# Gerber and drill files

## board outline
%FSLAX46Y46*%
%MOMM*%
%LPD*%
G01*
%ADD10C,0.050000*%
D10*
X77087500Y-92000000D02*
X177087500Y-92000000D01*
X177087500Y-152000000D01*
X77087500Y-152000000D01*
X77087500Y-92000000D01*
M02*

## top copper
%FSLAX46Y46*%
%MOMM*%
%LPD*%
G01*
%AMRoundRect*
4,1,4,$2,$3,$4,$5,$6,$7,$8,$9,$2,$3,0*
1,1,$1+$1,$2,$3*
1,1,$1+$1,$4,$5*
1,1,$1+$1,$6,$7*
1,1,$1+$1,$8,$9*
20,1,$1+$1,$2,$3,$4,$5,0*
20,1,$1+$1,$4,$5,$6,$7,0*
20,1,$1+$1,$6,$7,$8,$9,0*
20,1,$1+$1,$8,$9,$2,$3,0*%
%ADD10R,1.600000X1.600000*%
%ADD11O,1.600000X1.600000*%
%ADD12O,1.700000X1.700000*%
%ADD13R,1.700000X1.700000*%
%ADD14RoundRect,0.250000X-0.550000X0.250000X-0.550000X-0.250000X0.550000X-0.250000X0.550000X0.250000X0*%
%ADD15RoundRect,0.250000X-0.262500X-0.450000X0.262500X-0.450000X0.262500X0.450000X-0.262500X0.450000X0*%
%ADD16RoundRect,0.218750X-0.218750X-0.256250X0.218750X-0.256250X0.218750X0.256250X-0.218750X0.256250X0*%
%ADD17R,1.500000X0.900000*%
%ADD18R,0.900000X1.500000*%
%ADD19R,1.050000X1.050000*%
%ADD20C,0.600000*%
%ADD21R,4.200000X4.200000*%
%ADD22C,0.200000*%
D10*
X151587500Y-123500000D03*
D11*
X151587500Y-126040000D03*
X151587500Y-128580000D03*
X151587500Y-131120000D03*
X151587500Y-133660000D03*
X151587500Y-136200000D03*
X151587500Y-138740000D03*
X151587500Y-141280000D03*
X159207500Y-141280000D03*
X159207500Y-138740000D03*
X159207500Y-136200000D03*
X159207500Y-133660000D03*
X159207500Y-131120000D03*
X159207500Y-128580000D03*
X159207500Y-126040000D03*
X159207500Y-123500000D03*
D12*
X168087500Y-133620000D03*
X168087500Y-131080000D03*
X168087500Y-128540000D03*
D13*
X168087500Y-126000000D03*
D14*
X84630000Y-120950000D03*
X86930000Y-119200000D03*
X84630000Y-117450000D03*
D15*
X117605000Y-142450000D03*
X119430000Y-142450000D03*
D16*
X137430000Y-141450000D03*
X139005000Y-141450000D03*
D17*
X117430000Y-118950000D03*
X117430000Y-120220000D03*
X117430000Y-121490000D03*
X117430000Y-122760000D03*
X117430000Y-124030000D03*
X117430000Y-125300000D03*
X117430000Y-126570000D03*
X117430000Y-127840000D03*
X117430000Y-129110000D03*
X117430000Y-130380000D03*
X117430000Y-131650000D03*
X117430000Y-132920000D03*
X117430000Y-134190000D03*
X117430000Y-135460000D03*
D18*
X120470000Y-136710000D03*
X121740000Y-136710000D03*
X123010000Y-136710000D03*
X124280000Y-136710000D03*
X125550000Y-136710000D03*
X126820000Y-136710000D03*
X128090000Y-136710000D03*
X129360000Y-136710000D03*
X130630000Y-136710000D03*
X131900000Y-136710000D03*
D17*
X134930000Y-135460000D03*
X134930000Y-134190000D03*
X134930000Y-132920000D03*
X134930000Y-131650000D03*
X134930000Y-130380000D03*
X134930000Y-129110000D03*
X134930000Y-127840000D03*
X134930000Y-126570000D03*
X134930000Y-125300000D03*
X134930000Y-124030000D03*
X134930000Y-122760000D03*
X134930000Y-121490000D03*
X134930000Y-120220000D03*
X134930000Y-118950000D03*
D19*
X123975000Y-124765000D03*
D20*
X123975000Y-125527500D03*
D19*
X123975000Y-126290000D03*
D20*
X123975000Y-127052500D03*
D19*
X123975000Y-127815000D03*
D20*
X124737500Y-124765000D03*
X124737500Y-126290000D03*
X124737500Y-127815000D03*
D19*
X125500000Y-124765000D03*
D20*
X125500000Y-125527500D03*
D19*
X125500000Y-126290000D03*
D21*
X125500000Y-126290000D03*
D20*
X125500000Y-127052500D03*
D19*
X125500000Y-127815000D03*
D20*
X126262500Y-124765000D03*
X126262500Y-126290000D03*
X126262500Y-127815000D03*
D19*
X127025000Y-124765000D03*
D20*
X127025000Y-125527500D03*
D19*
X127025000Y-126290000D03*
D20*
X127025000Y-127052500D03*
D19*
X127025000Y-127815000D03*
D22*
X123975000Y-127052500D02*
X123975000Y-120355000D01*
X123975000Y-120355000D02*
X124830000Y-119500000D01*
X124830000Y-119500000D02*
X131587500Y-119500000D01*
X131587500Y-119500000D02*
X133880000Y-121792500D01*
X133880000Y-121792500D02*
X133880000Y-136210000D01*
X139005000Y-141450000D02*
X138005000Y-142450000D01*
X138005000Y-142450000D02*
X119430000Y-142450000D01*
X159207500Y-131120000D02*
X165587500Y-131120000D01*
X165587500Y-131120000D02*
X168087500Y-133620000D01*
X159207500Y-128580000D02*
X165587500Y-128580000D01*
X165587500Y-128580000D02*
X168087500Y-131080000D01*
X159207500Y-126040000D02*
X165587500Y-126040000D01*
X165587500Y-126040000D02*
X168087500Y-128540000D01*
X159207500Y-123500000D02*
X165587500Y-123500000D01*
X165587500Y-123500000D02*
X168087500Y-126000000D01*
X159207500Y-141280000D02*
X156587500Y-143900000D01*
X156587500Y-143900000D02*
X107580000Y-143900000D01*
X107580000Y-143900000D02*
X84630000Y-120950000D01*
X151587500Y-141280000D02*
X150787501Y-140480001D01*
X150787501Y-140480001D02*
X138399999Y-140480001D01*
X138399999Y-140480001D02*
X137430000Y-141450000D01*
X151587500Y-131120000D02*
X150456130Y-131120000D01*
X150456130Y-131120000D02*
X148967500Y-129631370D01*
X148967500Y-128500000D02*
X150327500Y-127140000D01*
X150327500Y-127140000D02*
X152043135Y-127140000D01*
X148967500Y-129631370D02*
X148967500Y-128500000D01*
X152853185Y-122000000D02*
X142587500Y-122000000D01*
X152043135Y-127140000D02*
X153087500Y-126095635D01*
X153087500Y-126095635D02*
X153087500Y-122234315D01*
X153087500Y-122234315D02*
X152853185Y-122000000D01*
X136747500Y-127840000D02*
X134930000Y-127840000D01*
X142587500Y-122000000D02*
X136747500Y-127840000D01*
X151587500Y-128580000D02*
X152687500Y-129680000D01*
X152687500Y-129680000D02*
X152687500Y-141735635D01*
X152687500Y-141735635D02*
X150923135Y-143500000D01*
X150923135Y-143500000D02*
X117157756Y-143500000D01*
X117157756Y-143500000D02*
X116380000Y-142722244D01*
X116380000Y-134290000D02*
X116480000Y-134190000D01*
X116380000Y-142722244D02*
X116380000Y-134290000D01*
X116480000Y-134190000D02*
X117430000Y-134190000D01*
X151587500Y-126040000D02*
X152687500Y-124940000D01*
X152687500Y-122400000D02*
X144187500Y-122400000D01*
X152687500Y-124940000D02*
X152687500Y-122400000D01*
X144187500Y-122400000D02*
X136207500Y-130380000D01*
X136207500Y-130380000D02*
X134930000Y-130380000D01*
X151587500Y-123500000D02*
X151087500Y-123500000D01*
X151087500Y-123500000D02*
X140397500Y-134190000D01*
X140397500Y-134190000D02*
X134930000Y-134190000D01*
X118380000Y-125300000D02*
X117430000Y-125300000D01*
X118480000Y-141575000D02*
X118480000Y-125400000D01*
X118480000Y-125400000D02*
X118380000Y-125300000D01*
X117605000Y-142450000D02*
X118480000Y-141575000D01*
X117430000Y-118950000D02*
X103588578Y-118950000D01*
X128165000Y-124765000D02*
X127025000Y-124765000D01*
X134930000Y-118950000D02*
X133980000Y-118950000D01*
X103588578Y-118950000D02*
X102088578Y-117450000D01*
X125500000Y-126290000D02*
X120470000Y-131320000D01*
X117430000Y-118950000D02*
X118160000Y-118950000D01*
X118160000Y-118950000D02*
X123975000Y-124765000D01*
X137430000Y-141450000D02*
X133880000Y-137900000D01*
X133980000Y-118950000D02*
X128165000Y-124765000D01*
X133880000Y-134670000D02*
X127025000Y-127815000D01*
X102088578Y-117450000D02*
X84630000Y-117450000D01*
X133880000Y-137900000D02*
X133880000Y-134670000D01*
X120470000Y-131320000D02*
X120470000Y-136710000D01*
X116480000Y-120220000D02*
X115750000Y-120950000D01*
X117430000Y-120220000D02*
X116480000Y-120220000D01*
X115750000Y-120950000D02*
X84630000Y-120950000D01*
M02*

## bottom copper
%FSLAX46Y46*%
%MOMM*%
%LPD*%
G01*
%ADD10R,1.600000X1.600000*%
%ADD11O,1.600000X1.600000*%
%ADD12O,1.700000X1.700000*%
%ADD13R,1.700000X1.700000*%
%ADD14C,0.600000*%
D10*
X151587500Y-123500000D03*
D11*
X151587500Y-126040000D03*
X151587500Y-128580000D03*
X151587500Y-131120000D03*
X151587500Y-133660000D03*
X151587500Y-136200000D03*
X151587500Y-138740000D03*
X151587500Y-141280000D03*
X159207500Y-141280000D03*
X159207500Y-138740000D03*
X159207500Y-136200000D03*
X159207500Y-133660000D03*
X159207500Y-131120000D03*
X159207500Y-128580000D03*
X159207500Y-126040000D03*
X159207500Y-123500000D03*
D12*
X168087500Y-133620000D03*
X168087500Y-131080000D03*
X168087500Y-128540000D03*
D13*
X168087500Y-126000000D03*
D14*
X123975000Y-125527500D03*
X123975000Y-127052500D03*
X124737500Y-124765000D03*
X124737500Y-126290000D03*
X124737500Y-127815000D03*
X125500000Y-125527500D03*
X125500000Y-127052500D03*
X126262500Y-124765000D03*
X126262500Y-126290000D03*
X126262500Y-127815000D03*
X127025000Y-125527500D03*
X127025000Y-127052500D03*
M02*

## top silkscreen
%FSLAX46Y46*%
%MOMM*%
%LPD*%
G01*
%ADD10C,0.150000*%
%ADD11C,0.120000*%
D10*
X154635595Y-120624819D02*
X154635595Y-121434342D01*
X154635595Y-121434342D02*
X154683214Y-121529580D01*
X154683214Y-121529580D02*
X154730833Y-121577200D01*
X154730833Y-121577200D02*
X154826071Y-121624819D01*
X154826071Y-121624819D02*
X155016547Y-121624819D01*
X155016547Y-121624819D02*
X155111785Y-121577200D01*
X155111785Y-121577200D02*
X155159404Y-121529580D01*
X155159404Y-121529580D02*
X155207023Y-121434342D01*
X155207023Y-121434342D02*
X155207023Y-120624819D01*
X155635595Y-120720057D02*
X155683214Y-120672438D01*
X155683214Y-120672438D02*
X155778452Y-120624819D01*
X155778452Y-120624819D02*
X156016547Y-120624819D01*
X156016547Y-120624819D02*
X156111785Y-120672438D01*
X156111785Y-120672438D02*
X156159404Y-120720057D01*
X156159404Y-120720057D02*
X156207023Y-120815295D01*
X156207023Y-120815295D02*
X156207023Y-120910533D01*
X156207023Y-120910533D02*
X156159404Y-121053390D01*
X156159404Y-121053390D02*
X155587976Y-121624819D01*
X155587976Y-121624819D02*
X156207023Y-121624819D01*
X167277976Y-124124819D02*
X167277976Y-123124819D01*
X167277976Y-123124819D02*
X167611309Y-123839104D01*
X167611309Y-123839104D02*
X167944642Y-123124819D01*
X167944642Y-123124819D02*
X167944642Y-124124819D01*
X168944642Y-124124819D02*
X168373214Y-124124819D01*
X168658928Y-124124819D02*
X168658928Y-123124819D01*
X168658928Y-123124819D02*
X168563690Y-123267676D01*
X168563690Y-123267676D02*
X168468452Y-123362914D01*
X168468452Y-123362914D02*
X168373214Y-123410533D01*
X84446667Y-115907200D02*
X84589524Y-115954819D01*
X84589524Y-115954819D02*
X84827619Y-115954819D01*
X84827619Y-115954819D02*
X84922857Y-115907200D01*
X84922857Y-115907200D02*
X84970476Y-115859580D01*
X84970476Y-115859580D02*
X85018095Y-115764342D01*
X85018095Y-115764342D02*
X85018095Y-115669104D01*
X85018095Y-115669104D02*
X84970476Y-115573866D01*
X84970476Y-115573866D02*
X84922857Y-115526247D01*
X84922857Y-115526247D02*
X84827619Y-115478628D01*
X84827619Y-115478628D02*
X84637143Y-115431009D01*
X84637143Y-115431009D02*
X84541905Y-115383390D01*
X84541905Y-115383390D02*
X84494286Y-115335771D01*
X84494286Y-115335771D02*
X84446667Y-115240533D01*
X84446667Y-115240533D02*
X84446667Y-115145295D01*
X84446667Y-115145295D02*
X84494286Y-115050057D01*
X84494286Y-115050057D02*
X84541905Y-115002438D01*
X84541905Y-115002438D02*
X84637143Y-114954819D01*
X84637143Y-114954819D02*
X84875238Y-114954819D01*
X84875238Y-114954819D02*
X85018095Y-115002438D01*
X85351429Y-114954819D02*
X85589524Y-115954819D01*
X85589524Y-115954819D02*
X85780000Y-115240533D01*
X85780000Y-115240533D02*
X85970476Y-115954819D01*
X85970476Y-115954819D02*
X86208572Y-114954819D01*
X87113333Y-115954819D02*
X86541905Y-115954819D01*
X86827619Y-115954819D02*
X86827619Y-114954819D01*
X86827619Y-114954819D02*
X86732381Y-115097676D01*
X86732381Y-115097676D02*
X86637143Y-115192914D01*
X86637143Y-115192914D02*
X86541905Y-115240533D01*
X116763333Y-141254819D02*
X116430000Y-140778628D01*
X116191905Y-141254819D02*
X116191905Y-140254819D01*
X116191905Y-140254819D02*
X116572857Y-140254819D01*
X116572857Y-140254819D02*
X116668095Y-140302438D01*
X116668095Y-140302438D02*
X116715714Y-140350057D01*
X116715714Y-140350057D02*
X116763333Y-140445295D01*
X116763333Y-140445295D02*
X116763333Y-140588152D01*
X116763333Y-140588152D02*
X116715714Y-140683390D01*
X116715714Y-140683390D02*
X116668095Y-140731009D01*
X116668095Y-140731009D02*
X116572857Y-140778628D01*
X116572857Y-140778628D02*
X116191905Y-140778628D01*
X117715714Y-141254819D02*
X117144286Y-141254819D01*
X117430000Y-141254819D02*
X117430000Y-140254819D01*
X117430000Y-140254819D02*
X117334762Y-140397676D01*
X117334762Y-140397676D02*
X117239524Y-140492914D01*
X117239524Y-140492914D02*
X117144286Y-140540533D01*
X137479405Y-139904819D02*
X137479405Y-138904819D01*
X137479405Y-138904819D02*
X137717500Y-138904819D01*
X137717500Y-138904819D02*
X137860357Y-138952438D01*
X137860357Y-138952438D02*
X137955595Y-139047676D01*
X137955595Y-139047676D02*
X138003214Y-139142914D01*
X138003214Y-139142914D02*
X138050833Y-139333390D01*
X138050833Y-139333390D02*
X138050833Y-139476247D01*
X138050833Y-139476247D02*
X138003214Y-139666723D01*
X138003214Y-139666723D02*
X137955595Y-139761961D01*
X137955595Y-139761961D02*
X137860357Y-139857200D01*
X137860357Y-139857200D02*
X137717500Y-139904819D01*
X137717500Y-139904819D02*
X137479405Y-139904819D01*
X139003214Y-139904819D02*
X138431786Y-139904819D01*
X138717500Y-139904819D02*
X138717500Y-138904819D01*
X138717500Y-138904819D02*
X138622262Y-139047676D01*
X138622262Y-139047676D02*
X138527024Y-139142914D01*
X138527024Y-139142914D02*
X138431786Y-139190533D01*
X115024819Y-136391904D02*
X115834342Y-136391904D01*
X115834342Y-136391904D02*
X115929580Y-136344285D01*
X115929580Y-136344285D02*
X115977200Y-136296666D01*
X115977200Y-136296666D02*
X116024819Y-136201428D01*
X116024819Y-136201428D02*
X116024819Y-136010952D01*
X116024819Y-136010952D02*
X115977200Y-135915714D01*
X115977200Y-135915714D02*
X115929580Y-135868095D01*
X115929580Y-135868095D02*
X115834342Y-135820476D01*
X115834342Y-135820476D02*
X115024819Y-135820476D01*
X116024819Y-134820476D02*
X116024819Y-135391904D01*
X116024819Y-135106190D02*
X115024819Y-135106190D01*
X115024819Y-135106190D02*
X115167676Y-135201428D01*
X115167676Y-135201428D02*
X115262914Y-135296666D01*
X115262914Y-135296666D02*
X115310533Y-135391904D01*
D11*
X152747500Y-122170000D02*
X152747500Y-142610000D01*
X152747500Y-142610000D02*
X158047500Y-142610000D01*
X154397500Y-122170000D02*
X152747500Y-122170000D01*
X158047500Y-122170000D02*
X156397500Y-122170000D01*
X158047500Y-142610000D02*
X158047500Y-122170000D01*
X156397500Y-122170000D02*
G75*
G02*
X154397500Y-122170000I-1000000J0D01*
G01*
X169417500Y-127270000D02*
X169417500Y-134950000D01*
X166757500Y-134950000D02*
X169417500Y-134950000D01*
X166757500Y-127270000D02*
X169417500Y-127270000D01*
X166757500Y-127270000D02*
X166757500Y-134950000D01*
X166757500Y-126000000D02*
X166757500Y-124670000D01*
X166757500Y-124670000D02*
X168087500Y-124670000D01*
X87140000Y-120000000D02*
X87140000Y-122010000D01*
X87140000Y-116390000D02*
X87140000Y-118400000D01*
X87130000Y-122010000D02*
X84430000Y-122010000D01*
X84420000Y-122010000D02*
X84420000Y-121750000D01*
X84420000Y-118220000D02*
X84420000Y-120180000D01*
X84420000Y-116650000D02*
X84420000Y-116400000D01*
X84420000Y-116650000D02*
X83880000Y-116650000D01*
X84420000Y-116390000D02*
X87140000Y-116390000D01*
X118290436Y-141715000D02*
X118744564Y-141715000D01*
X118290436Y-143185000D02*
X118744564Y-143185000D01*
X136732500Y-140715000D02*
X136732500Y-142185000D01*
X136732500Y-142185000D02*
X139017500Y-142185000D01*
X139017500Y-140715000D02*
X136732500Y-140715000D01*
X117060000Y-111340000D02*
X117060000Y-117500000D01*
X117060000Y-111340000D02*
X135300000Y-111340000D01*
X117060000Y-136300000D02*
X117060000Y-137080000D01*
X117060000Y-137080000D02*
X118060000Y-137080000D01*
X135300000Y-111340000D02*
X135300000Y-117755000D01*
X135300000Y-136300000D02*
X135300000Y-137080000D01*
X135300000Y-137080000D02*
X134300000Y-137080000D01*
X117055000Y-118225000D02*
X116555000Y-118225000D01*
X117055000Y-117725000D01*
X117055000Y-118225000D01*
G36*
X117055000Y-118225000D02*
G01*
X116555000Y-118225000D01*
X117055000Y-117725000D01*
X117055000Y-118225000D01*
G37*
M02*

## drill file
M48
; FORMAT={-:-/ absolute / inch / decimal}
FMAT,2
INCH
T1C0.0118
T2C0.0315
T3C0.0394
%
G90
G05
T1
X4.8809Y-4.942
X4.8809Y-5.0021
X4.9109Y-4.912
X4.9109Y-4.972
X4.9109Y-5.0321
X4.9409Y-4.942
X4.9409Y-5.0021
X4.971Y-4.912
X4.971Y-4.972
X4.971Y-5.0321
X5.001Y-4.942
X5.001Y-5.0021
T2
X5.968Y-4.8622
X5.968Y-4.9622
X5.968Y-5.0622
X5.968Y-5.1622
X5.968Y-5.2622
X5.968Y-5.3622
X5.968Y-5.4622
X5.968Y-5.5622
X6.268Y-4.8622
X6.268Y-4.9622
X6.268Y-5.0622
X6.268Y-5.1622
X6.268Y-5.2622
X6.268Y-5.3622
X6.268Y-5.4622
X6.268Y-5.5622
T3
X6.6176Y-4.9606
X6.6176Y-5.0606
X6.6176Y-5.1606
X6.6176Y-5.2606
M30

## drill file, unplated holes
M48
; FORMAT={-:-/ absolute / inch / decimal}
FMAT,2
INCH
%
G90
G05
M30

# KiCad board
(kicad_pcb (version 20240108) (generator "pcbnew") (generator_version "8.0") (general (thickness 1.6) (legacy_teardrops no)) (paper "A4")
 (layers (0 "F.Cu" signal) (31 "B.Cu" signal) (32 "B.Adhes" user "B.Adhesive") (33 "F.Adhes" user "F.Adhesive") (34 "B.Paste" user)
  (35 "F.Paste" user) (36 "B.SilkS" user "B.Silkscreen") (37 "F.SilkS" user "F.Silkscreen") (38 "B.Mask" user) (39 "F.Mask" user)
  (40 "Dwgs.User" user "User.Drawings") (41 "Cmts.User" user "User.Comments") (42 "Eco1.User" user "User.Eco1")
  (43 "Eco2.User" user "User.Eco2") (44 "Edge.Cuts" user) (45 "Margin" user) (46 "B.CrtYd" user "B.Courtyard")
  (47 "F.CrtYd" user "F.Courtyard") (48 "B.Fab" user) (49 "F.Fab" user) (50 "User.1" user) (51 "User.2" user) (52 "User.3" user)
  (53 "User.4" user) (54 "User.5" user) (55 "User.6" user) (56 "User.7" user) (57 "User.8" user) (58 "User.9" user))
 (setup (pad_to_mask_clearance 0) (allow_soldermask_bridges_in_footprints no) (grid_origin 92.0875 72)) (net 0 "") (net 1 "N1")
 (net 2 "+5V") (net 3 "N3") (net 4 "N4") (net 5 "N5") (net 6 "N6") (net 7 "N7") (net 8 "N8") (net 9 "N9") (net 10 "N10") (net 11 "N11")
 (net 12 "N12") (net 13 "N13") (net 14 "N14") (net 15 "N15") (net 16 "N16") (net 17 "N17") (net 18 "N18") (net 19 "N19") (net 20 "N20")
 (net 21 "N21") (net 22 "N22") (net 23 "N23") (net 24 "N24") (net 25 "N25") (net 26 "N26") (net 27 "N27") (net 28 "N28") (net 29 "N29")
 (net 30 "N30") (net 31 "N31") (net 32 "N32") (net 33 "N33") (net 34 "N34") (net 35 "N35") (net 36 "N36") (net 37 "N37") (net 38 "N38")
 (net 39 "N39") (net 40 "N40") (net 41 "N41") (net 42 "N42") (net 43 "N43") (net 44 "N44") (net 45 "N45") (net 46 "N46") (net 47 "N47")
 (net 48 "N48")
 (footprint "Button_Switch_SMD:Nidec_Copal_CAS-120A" (layer "F.Cu") (at 85.78 119.2)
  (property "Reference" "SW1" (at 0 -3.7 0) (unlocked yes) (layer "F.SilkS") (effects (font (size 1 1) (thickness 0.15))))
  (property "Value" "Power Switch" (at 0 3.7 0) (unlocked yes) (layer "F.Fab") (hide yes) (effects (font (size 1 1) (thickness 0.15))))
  (fp_line (start -1.36 -2.81) (end 1.36 -2.81) (stroke (width 0.12) (type solid)) (layer "F.SilkS"))
  (fp_line (start -1.36 -2.55) (end -1.9 -2.55) (stroke (width 0.12) (type default)) (layer "F.SilkS"))
  (fp_line (start -1.36 -2.55) (end -1.36 -2.8) (stroke (width 0.12) (type solid)) (layer "F.SilkS"))
  (fp_line (start -1.36 -0.98) (end -1.36 0.98) (stroke (width 0.12) (type solid)) (layer "F.SilkS"))
  (fp_line (start -1.36 2.81) (end -1.36 2.55) (stroke (width 0.12) (type solid)) (layer "F.SilkS"))
  (fp_line (start 1.35 2.81) (end -1.35 2.81) (stroke (width 0.12) (type solid)) (layer "F.SilkS"))
  (fp_line (start 1.36 -2.81) (end 1.36 -0.8) (stroke (width 0.12) (type solid)) (layer "F.SilkS"))
  (fp_line (start 1.36 0.8) (end 1.36 2.81) (stroke (width 0.12) (type solid)) (layer "F.SilkS"))
  (pad "1" smd roundrect (at -1.15 -1.75 270) (size 1 1.6) (layers "F.Cu" "F.Paste" "F.Mask") (roundrect_rratio 0.25) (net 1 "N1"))
  (pad "2" smd roundrect (at 1.15 0 270) (size 1 1.6) (layers "F.Cu" "F.Paste" "F.Mask") (roundrect_rratio 0.25) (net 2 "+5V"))
  (pad "3" smd roundrect (at -1.15 1.75 270) (size 1 1.6) (layers "F.Cu" "F.Paste" "F.Mask") (roundrect_rratio 0.25) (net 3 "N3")))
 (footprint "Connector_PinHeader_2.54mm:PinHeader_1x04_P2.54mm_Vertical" (layer "F.Cu") (at 168.0875 126)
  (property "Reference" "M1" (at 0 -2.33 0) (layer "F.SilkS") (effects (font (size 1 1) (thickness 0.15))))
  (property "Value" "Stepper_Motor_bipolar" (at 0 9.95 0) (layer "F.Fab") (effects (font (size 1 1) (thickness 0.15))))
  (fp_line (start -1.33 -1.33) (end 0 -1.33) (stroke (width 0.12) (type solid)) (layer "F.SilkS"))
  (fp_line (start -1.33 0) (end -1.33 -1.33) (stroke (width 0.12) (type solid)) (layer "F.SilkS"))
  (fp_line (start -1.33 1.27) (end -1.33 8.95) (stroke (width 0.12) (type solid)) (layer "F.SilkS"))
  (fp_line (start -1.33 1.27) (end 1.33 1.27) (stroke (width 0.12) (type solid)) (layer "F.SilkS"))
  (fp_line (start -1.33 8.95) (end 1.33 8.95) (stroke (width 0.12) (type solid)) (layer "F.SilkS"))
  (fp_line (start 1.33 1.27) (end 1.33 8.95) (stroke (width 0.12) (type solid)) (layer "F.SilkS"))
  (pad "1" thru_hole rect (at 0 0) (size 1.7 1.7) (drill 1) (layers "*.Cu" "*.Mask") (remove_unused_layers no) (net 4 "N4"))
  (pad "2" thru_hole oval (at 0 2.54) (size 1.7 1.7) (drill 1) (layers "*.Cu" "*.Mask") (remove_unused_layers no) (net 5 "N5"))
  (pad "3" thru_hole oval (at 0 5.08) (size 1.7 1.7) (drill 1) (layers "*.Cu" "*.Mask") (remove_unused_layers no) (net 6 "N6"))
  (pad "4" thru_hole oval (at 0 7.62) (size 1.7 1.7) (drill 1) (layers "*.Cu" "*.Mask") (remove_unused_layers no) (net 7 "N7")))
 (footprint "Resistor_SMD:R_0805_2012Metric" (layer "F.Cu") (at 118.5175 142.45)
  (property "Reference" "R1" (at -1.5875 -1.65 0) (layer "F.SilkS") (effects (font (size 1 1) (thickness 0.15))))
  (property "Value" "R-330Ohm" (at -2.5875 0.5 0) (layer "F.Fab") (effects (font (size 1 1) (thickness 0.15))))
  (fp_line (start -0.227064 -0.735) (end 0.227064 -0.735) (stroke (width 0.12) (type solid)) (layer "F.SilkS"))
  (fp_line (start -0.227064 0.735) (end 0.227064 0.735) (stroke (width 0.12) (type solid)) (layer "F.SilkS"))
  (pad "1" smd roundrect (at -0.9125 0) (size 1.025 1.4) (layers "F.Cu" "F.Paste" "F.Mask") (roundrect_rratio 0.243902) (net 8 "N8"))
  (pad "2" smd roundrect (at 0.9125 0) (size 1.025 1.4) (layers "F.Cu" "F.Paste" "F.Mask") (roundrect_rratio 0.243902) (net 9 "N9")))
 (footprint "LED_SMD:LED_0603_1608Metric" (layer "F.Cu") (at 138.2175 141.45)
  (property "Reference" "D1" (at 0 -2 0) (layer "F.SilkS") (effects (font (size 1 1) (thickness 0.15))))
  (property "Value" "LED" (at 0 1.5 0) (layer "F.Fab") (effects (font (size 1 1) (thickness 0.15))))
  (fp_line (start -1.485 -0.735) (end -1.485 0.735) (stroke (width 0.12) (type solid)) (layer "F.SilkS"))
  (fp_line (start -1.485 0.735) (end 0.8 0.735) (stroke (width 0.12) (type solid)) (layer "F.SilkS"))
  (fp_line (start 0.8 -0.735) (end -1.485 -0.735) (stroke (width 0.12) (type solid)) (layer "F.SilkS"))
  (pad "1" smd roundrect (at -0.7875 0) (size 0.875 0.95) (layers "F.Cu" "F.Paste" "F.Mask") (roundrect_rratio 0.25) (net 1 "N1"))
  (pad "2" smd roundrect (at 0.7875 0) (size 0.875 0.95) (layers "F.Cu" "F.Paste" "F.Mask") (roundrect_rratio 0.25) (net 9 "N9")))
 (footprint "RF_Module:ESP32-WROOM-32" (layer "F.Cu") (at 126.18 127.2)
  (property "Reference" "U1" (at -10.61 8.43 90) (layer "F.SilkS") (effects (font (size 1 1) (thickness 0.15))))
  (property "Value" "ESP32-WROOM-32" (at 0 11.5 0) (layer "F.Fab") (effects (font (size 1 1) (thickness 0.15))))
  (fp_line (start -9.12 -15.86) (end -9.12 -9.7) (stroke (width 0.12) (type solid)) (layer "F.SilkS"))
  (fp_line (start -9.12 -15.86) (end 9.12 -15.86) (stroke (width 0.12) (type solid)) (layer "F.SilkS"))
  (fp_line (start -9.12 9.1) (end -9.12 9.88) (stroke (width 0.12) (type solid)) (layer "F.SilkS"))
  (fp_line (start -9.12 9.88) (end -8.12 9.88) (stroke (width 0.12) (type solid)) (layer "F.SilkS"))
  (fp_line (start 9.12 -15.86) (end 9.12 -9.445) (stroke (width 0.12) (type solid)) (layer "F.SilkS"))
  (fp_line (start 9.12 9.1) (end 9.12 9.88) (stroke (width 0.12) (type solid)) (layer "F.SilkS"))
  (fp_line (start 9.12 9.88) (end 8.12 9.88) (stroke (width 0.12) (type solid)) (layer "F.SilkS"))
  (fp_poly
   (pts (xy -9.125 -8.975) (xy -9.625 -8.975) (xy -9.125 -9.475) (xy -9.125 -8.975)) (stroke (width 0.12) (type solid)) (fill solid)
   (layer "F.SilkS"))
  (pad "1" smd rect (at -8.75 -8.25) (size 1.5 0.9) (layers "F.Cu" "F.Paste" "F.Mask") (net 1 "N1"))
  (pad "2" smd rect (at -8.75 -6.98) (size 1.5 0.9) (layers "F.Cu" "F.Paste" "F.Mask") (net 3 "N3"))
  (pad "3" smd rect (at -8.75 -5.71) (size 1.5 0.9) (layers "F.Cu" "F.Paste" "F.Mask") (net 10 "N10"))
  (pad "4" smd rect (at -8.75 -4.44) (size 1.5 0.9) (layers "F.Cu" "F.Paste" "F.Mask") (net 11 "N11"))
  (pad "5" smd rect (at -8.75 -3.17) (size 1.5 0.9) (layers "F.Cu" "F.Paste" "F.Mask") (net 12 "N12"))
  (pad "6" smd rect (at -8.75 -1.9) (size 1.5 0.9) (layers "F.Cu" "F.Paste" "F.Mask") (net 8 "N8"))
  (pad "7" smd rect (at -8.75 -0.63) (size 1.5 0.9) (layers "F.Cu" "F.Paste" "F.Mask") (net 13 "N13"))
  (pad "8" smd rect (at -8.75 0.64) (size 1.5 0.9) (layers "F.Cu" "F.Paste" "F.Mask") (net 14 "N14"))
  (pad "9" smd rect (at -8.75 1.91) (size 1.5 0.9) (layers "F.Cu" "F.Paste" "F.Mask") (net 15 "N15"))
  (pad "10" smd rect (at -8.75 3.18) (size 1.5 0.9) (layers "F.Cu" "F.Paste" "F.Mask") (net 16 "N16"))
  (pad "11" smd rect (at -8.75 4.45) (size 1.5 0.9) (layers "F.Cu" "F.Paste" "F.Mask") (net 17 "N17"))
  (pad "12" smd rect (at -8.75 5.72) (size 1.5 0.9) (layers "F.Cu" "F.Paste" "F.Mask") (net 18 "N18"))
  (pad "13" smd rect (at -8.75 6.99) (size 1.5 0.9) (layers "F.Cu" "F.Paste" "F.Mask") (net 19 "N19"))
  (pad "14" smd rect (at -8.75 8.26) (size 1.5 0.9) (layers "F.Cu" "F.Paste" "F.Mask") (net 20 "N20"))
  (pad "15" smd rect (at -5.71 9.51 90) (size 1.5 0.9) (layers "F.Cu" "F.Paste" "F.Mask") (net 1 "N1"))
  (pad "16" smd rect (at -4.44 9.51 90) (size 1.5 0.9) (layers "F.Cu" "F.Paste" "F.Mask") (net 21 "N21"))
  (pad "17" smd rect (at -3.17 9.51 90) (size 1.5 0.9) (layers "F.Cu" "F.Paste" "F.Mask") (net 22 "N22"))
  (pad "18" smd rect (at -1.9 9.51 90) (size 1.5 0.9) (layers "F.Cu" "F.Paste" "F.Mask") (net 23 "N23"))
  (pad "19" smd rect (at -0.63 9.51 90) (size 1.5 0.9) (layers "F.Cu" "F.Paste" "F.Mask") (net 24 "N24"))
  (pad "20" smd rect (at 0.64 9.51 90) (size 1.5 0.9) (layers "F.Cu" "F.Paste" "F.Mask") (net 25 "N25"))
  (pad "21" smd rect (at 1.91 9.51 90) (size 1.5 0.9) (layers "F.Cu" "F.Paste" "F.Mask") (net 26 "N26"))
  (pad "22" smd rect (at 3.18 9.51 90) (size 1.5 0.9) (layers "F.Cu" "F.Paste" "F.Mask") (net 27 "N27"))
  (pad "23" smd rect (at 4.45 9.51 90) (size 1.5 0.9) (layers "F.Cu" "F.Paste" "F.Mask") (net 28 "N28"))
  (pad "24" smd rect (at 5.72 9.51 90) (size 1.5 0.9) (layers "F.Cu" "F.Paste" "F.Mask") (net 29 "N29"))
  (pad "25" smd rect (at 8.75 8.26) (size 1.5 0.9) (layers "F.Cu" "F.Paste" "F.Mask") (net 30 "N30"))
  (pad "26" smd rect (at 8.75 6.99) (size 1.5 0.9) (layers "F.Cu" "F.Paste" "F.Mask") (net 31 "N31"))
  (pad "27" smd rect (at 8.75 5.72) (size 1.5 0.9) (layers "F.Cu" "F.Paste" "F.Mask") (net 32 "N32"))
  (pad "28" smd rect (at 8.75 4.45) (size 1.5 0.9) (layers "F.Cu" "F.Paste" "F.Mask") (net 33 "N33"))
  (pad "29" smd rect (at 8.75 3.18) (size 1.5 0.9) (layers "F.Cu" "F.Paste" "F.Mask") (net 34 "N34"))
  (pad "30" smd rect (at 8.75 1.91) (size 1.5 0.9) (layers "F.Cu" "F.Paste" "F.Mask") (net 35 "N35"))
  (pad "31" smd rect (at 8.75 0.64) (size 1.5 0.9) (layers "F.Cu" "F.Paste" "F.Mask") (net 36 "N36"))
  (pad "32" smd rect (at 8.75 -0.63) (size 1.5 0.9) (layers "F.Cu" "F.Paste" "F.Mask") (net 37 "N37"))
  (pad "33" smd rect (at 8.75 -1.9) (size 1.5 0.9) (layers "F.Cu" "F.Paste" "F.Mask") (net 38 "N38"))
  (pad "34" smd rect (at 8.75 -3.17) (size 1.5 0.9) (layers "F.Cu" "F.Paste" "F.Mask") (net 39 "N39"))
  (pad "35" smd rect (at 8.75 -4.44) (size 1.5 0.9) (layers "F.Cu" "F.Paste" "F.Mask") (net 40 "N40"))
  (pad "36" smd rect (at 8.75 -5.71) (size 1.5 0.9) (layers "F.Cu" "F.Paste" "F.Mask") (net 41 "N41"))
  (pad "37" smd rect (at 8.75 -6.98) (size 1.5 0.9) (layers "F.Cu" "F.Paste" "F.Mask") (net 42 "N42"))
  (pad "38" smd rect (at 8.75 -8.25) (size 1.5 0.9) (layers "F.Cu" "F.Paste" "F.Mask") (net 1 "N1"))
  (pad "39" smd rect (at -2.205 -2.435) (size 1.05 1.05) (layers "F.Cu" "F.Paste") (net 1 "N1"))
  (pad "39" thru_hole circle (at -2.205 -1.6725) (size 0.6 0.6) (drill 0.3) (layers "*.Cu" "F.Mask") (remove_unused_layers no) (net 1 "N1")
   (zone_connect 2))
  (pad "39" smd rect (at -2.205 -0.91) (size 1.05 1.05) (layers "F.Cu" "F.Paste") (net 1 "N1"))
  (pad "39" thru_hole circle (at -2.205 -0.1475) (size 0.6 0.6) (drill 0.3) (layers "*.Cu" "F.Mask") (remove_unused_layers no) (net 1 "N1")
   (zone_connect 2))
  (pad "39" smd rect (at -2.205 0.615) (size 1.05 1.05) (layers "F.Cu" "F.Paste") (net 1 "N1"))
  (pad "39" thru_hole circle (at -1.4425 -2.435) (size 0.6 0.6) (drill 0.3) (layers "*.Cu" "F.Mask") (remove_unused_layers no) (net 1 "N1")
   (zone_connect 2))
  (pad "39" thru_hole circle (at -1.4425 -0.91) (size 0.6 0.6) (drill 0.3) (layers "*.Cu" "F.Mask") (remove_unused_layers no) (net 1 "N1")
   (zone_connect 2))
  (pad "39" thru_hole circle (at -1.4425 0.615) (size 0.6 0.6) (drill 0.3) (layers "*.Cu" "F.Mask") (remove_unused_layers no) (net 1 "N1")
   (zone_connect 2))
  (pad "39" smd rect (at -0.68 -2.435) (size 1.05 1.05) (layers "F.Cu" "F.Paste") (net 1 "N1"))
  (pad "39" thru_hole circle (at -0.68 -1.6725) (size 0.6 0.6) (drill 0.3) (layers "*.Cu" "F.Mask") (remove_unused_layers no) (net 1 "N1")
   (zone_connect 2))
  (pad "39" smd rect (at -0.68 -0.91) (size 1.05 1.05) (layers "F.Cu" "F.Paste") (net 1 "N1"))
  (pad "39" smd rect (at -0.68 -0.91) (size 4.2 4.2) (layers "F.Cu" "F.Mask") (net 1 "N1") (zone_connect 2))
  (pad "39" thru_hole circle (at -0.68 -0.1475) (size 0.6 0.6) (drill 0.3) (layers "*.Cu" "F.Mask") (remove_unused_layers no) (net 1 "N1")
   (zone_connect 2))
  (pad "39" smd rect (at -0.68 0.615) (size 1.05 1.05) (layers "F.Cu" "F.Paste") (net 1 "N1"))
  (pad "39" thru_hole circle (at 0.0825 -2.435) (size 0.6 0.6) (drill 0.3) (layers "*.Cu" "F.Mask") (remove_unused_layers no) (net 1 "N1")
   (zone_connect 2))
  (pad "39" thru_hole circle (at 0.0825 -0.91) (size 0.6 0.6) (drill 0.3) (layers "*.Cu" "F.Mask") (remove_unused_layers no) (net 1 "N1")
   (zone_connect 2))
  (pad "39" thru_hole circle (at 0.0825 0.615) (size 0.6 0.6) (drill 0.3) (layers "*.Cu" "F.Mask") (remove_unused_layers no) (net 1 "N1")
   (zone_connect 2))
  (pad "39" smd rect (at 0.845 -2.435) (size 1.05 1.05) (layers "F.Cu" "F.Paste") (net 1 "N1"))
  (pad "39" thru_hole circle (at 0.845 -1.6725) (size 0.6 0.6) (drill 0.3) (layers "*.Cu" "F.Mask") (remove_unused_layers no) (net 1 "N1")
   (zone_connect 2))
  (pad "39" smd rect (at 0.845 -0.91) (size 1.05 1.05) (layers "F.Cu" "F.Paste") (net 1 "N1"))
  (pad "39" thru_hole circle (at 0.845 -0.1475) (size 0.6 0.6) (drill 0.3) (layers "*.Cu" "F.Mask") (remove_unused_layers no) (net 1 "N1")
   (zone_connect 2))
  (pad "39" smd rect (at 0.845 0.615) (size 1.05 1.05) (layers "F.Cu" "F.Paste") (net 1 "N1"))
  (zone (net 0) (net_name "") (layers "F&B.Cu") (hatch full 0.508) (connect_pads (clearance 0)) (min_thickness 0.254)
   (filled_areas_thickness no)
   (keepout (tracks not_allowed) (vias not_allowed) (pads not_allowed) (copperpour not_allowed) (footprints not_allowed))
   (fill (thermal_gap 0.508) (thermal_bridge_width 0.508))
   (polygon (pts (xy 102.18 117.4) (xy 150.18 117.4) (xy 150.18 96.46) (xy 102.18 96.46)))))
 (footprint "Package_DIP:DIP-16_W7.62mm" (layer "F.Cu") (at 151.5875 123.5)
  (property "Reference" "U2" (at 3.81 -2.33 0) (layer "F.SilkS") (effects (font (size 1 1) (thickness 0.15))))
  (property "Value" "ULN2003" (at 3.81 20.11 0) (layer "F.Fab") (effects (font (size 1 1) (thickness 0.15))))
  (fp_line (start 1.16 -1.33) (end 1.16 19.11) (stroke (width 0.12) (type solid)) (layer "F.SilkS"))
  (fp_line (start 1.16 19.11) (end 6.46 19.11) (stroke (width 0.12) (type solid)) (layer "F.SilkS"))
  (fp_line (start 2.81 -1.33) (end 1.16 -1.33) (stroke (width 0.12) (type solid)) (layer "F.SilkS"))
  (fp_line (start 6.46 -1.33) (end 4.81 -1.33) (stroke (width 0.12) (type solid)) (layer "F.SilkS"))
  (fp_line (start 6.46 19.11) (end 6.46 -1.33) (stroke (width 0.12) (type solid)) (layer "F.SilkS"))
  (fp_arc (start 4.81 -1.33) (mid 3.81 -0.33) (end 2.81 -1.33) (stroke (width 0.12) (type solid)) (layer "F.SilkS"))
  (pad "1" thru_hole rect (at 0 0) (size 1.6 1.6) (drill 0.8) (layers "*.Cu" "*.Mask") (remove_unused_layers no) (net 31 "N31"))
  (pad "2" thru_hole oval (at 0 2.54) (size 1.6 1.6) (drill 0.8) (layers "*.Cu" "*.Mask") (remove_unused_layers no) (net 34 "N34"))
  (pad "3" thru_hole oval (at 0 5.08) (size 1.6 1.6) (drill 0.8) (layers "*.Cu" "*.Mask") (remove_unused_layers no) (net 19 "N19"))
  (pad "4" thru_hole oval (at 0 7.62) (size 1.6 1.6) (drill 0.8) (layers "*.Cu" "*.Mask") (remove_unused_layers no) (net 36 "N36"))
  (pad "5" thru_hole oval (at 0 10.16) (size 1.6 1.6) (drill 0.8) (layers "*.Cu" "*.Mask") (remove_unused_layers no) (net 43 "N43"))
  (pad "6" thru_hole oval (at 0 12.7) (size 1.6 1.6) (drill 0.8) (layers "*.Cu" "*.Mask") (remove_unused_layers no) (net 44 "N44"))
  (pad "7" thru_hole oval (at 0 15.24) (size 1.6 1.6) (drill 0.8) (layers "*.Cu" "*.Mask") (remove_unused_layers no) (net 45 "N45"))
  (pad "8" thru_hole oval (at 0 17.78) (size 1.6 1.6) (drill 0.8) (layers "*.Cu" "*.Mask") (remove_unused_layers no) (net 1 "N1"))
  (pad "9" thru_hole oval (at 7.62 17.78) (size 1.6 1.6) (drill 0.8) (layers "*.Cu" "*.Mask") (remove_unused_layers no) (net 3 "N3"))
  (pad "10" thru_hole oval (at 7.62 15.24) (size 1.6 1.6) (drill 0.8) (layers "*.Cu" "*.Mask") (remove_unused_layers no) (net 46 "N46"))
  (pad "11" thru_hole oval (at 7.62 12.7) (size 1.6 1.6) (drill 0.8) (layers "*.Cu" "*.Mask") (remove_unused_layers no) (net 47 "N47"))
  (pad "12" thru_hole oval (at 7.62 10.16) (size 1.6 1.6) (drill 0.8) (layers "*.Cu" "*.Mask") (remove_unused_layers no) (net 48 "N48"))
  (pad "13" thru_hole oval (at 7.62 7.62) (size 1.6 1.6) (drill 0.8) (layers "*.Cu" "*.Mask") (remove_unused_layers no) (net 7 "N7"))
  (pad "14" thru_hole oval (at 7.62 5.08) (size 1.6 1.6) (drill 0.8) (layers "*.Cu" "*.Mask") (remove_unused_layers no) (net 6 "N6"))
  (pad "15" thru_hole oval (at 7.62 2.54) (size 1.6 1.6) (drill 0.8) (layers "*.Cu" "*.Mask") (remove_unused_layers no) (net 5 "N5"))
  (pad "16" thru_hole oval (at 7.62 0) (size 1.6 1.6) (drill 0.8) (layers "*.Cu" "*.Mask") (remove_unused_layers no) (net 4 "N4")))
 (gr_rect (start 77.0875 92) (end 177.0875 152) (stroke (width 0.05) (type default)) (fill none) (layer "Edge.Cuts"))
 (segment (start 118.38 125.3) (end 117.43 125.3) (width 0.2) (layer "F.Cu") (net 8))
 (segment (start 118.48 141.575) (end 118.48 125.4) (width 0.2) (layer "F.Cu") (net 8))
 (segment (start 118.48 125.4) (end 118.38 125.3) (width 0.2) (layer "F.Cu") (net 8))
 (segment (start 117.605 142.45) (end 118.48 141.575) (width 0.2) (layer "F.Cu") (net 8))
 (segment (start 138.005 142.45) (end 119.43 142.45) (width 0.2) (layer "F.Cu") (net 9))
 (segment (start 139.005 141.45) (end 138.005 142.45) (width 0.2) (layer "F.Cu") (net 9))
 (segment (start 124.83 119.5) (end 131.5875 119.5) (width 0.2) (layer "F.Cu") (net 1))
 (segment (start 117.43 118.95) (end 103.588578 118.95) (width 0.2) (layer "F.Cu") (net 1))
 (segment (start 138.399999 140.480001) (end 137.43 141.45) (width 0.2) (layer "F.Cu") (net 1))
 (segment (start 123.975 127.0525) (end 123.975 120.355) (width 0.2) (layer "F.Cu") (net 1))
 (segment (start 128.165 124.765) (end 127.025 124.765) (width 0.2) (layer "F.Cu") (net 1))
 (segment (start 134.93 118.95) (end 133.98 118.95) (width 0.2) (layer "F.Cu") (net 1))
 (segment (start 133.88 121.7925) (end 133.88 136.21) (width 0.2) (layer "F.Cu") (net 1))
 (segment (start 151.5875 141.28) (end 150.787501 140.480001) (width 0.2) (layer "F.Cu") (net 1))
 (segment (start 103.588578 118.95) (end 102.088578 117.45) (width 0.2) (layer "F.Cu") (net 1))
 (segment (start 125.5 126.29) (end 120.47 131.32) (width 0.2) (layer "F.Cu") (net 1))
 (segment (start 123.975 120.355) (end 124.83 119.5) (width 0.2) (layer "F.Cu") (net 1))
 (segment (start 117.43 118.95) (end 118.16 118.95) (width 0.2) (layer "F.Cu") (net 1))
 (segment (start 150.787501 140.480001) (end 138.399999 140.480001) (width 0.2) (layer "F.Cu") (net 1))
 (segment (start 118.16 118.95) (end 123.975 124.765) (width 0.2) (layer "F.Cu") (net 1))
 (segment (start 137.43 141.45) (end 133.88 137.9) (width 0.2) (layer "F.Cu") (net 1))
 (segment (start 133.98 118.95) (end 128.165 124.765) (width 0.2) (layer "F.Cu") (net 1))
 (segment (start 133.88 134.67) (end 127.025 127.815) (width 0.2) (layer "F.Cu") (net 1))
 (segment (start 102.088578 117.45) (end 84.63 117.45) (width 0.2) (layer "F.Cu") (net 1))
 (segment (start 131.5875 119.5) (end 133.88 121.7925) (width 0.2) (layer "F.Cu") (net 1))
 (segment (start 133.88 137.9) (end 133.88 134.67) (width 0.2) (layer "F.Cu") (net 1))
 (segment (start 120.47 131.32) (end 120.47 136.71) (width 0.2) (layer "F.Cu") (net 1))
 (segment (start 116.48 120.22) (end 115.75 120.95) (width 0.2) (layer "F.Cu") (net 3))
 (segment (start 156.5875 143.9) (end 107.58 143.9) (width 0.2) (layer "F.Cu") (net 3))
 (segment (start 107.58 143.9) (end 84.63 120.95) (width 0.2) (layer "F.Cu") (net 3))
 (segment (start 159.2075 141.28) (end 156.5875 143.9) (width 0.2) (layer "F.Cu") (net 3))
 (segment (start 117.43 120.22) (end 116.48 120.22) (width 0.2) (layer "F.Cu") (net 3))
 (segment (start 115.75 120.95) (end 84.63 120.95) (width 0.2) (layer "F.Cu") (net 3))
 (segment (start 151.5875 126.04) (end 152.6875 124.94) (width 0.2) (layer "F.Cu") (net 34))
 (segment (start 136.2075 130.38) (end 134.93 130.38) (width 0.2) (layer "F.Cu") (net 34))
 (segment (start 152.6875 122.4) (end 144.1875 122.4) (width 0.2) (layer "F.Cu") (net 34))
 (segment (start 144.1875 122.4) (end 136.2075 130.38) (width 0.2) (layer "F.Cu") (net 34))
 (segment (start 152.6875 124.94) (end 152.6875 122.4) (width 0.2) (layer "F.Cu") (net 34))
 (segment (start 148.9675 129.63137) (end 148.9675 128.5) (width 0.2) (layer "F.Cu") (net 36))
 (segment (start 150.3275 127.14) (end 152.043135 127.14) (width 0.2) (layer "F.Cu") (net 36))
 (segment (start 142.5875 122) (end 136.7475 127.84) (width 0.2) (layer "F.Cu") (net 36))
 (segment (start 136.7475 127.84) (end 134.93 127.84) (width 0.2) (layer "F.Cu") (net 36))
 (segment (start 153.0875 126.095635) (end 153.0875 122.234315) (width 0.2) (layer "F.Cu") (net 36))
 (segment (start 152.853185 122) (end 142.5875 122) (width 0.2) (layer "F.Cu") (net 36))
 (segment (start 152.043135 127.14) (end 153.0875 126.095635) (width 0.2) (layer "F.Cu") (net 36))
 (segment (start 153.0875 122.234315) (end 152.853185 122) (width 0.2) (layer "F.Cu") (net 36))
 (segment (start 151.5875 131.12) (end 150.45613 131.12) (width 0.2) (layer "F.Cu") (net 36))
 (segment (start 150.45613 131.12) (end 148.9675 129.63137) (width 0.2) (layer "F.Cu") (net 36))
 (segment (start 148.9675 128.5) (end 150.3275 127.14) (width 0.2) (layer "F.Cu") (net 36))
 (segment (start 150.923135 143.5) (end 117.157756 143.5) (width 0.2) (layer "F.Cu") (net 19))
 (segment (start 152.6875 129.68) (end 152.6875 141.735635) (width 0.2) (layer "F.Cu") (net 19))
 (segment (start 116.38 134.29) (end 116.48 134.19) (width 0.2) (layer "F.Cu") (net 19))
 (segment (start 151.5875 128.58) (end 152.6875 129.68) (width 0.2) (layer "F.Cu") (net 19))
 (segment (start 116.38 142.722244) (end 116.38 134.29) (width 0.2) (layer "F.Cu") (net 19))
 (segment (start 152.6875 141.735635) (end 150.923135 143.5) (width 0.2) (layer "F.Cu") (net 19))
 (segment (start 117.157756 143.5) (end 116.38 142.722244) (width 0.2) (layer "F.Cu") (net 19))
 (segment (start 116.48 134.19) (end 117.43 134.19) (width 0.2) (layer "F.Cu") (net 19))
 (segment (start 151.0875 123.5) (end 140.3975 134.19) (width 0.2) (layer "F.Cu") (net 31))
 (segment (start 151.5875 123.5) (end 151.0875 123.5) (width 0.2) (layer "F.Cu") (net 31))
 (segment (start 140.3975 134.19) (end 134.93 134.19) (width 0.2) (layer "F.Cu") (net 31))
 (segment (start 159.2075 131.12) (end 165.5875 131.12) (width 0.2) (layer "F.Cu") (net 7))
 (segment (start 165.5875 131.12) (end 168.0875 133.62) (width 0.2) (layer "F.Cu") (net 7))
 (segment (start 159.2075 123.5) (end 165.5875 123.5) (width 0.2) (layer "F.Cu") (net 4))
 (segment (start 165.5875 123.5) (end 168.0875 126) (width 0.2) (layer "F.Cu") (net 4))
 (segment (start 165.5875 126.04) (end 168.0875 128.54) (width 0.2) (layer "F.Cu") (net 5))
 (segment (start 159.2075 126.04) (end 165.5875 126.04) (width 0.2) (layer "F.Cu") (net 5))
 (segment (start 165.5875 128.58) (end 168.0875 131.08) (width 0.2) (layer "F.Cu") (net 6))
 (segment (start 159.2075 128.58) (end 165.5875 128.58) (width 0.2) (layer "F.Cu") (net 6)))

